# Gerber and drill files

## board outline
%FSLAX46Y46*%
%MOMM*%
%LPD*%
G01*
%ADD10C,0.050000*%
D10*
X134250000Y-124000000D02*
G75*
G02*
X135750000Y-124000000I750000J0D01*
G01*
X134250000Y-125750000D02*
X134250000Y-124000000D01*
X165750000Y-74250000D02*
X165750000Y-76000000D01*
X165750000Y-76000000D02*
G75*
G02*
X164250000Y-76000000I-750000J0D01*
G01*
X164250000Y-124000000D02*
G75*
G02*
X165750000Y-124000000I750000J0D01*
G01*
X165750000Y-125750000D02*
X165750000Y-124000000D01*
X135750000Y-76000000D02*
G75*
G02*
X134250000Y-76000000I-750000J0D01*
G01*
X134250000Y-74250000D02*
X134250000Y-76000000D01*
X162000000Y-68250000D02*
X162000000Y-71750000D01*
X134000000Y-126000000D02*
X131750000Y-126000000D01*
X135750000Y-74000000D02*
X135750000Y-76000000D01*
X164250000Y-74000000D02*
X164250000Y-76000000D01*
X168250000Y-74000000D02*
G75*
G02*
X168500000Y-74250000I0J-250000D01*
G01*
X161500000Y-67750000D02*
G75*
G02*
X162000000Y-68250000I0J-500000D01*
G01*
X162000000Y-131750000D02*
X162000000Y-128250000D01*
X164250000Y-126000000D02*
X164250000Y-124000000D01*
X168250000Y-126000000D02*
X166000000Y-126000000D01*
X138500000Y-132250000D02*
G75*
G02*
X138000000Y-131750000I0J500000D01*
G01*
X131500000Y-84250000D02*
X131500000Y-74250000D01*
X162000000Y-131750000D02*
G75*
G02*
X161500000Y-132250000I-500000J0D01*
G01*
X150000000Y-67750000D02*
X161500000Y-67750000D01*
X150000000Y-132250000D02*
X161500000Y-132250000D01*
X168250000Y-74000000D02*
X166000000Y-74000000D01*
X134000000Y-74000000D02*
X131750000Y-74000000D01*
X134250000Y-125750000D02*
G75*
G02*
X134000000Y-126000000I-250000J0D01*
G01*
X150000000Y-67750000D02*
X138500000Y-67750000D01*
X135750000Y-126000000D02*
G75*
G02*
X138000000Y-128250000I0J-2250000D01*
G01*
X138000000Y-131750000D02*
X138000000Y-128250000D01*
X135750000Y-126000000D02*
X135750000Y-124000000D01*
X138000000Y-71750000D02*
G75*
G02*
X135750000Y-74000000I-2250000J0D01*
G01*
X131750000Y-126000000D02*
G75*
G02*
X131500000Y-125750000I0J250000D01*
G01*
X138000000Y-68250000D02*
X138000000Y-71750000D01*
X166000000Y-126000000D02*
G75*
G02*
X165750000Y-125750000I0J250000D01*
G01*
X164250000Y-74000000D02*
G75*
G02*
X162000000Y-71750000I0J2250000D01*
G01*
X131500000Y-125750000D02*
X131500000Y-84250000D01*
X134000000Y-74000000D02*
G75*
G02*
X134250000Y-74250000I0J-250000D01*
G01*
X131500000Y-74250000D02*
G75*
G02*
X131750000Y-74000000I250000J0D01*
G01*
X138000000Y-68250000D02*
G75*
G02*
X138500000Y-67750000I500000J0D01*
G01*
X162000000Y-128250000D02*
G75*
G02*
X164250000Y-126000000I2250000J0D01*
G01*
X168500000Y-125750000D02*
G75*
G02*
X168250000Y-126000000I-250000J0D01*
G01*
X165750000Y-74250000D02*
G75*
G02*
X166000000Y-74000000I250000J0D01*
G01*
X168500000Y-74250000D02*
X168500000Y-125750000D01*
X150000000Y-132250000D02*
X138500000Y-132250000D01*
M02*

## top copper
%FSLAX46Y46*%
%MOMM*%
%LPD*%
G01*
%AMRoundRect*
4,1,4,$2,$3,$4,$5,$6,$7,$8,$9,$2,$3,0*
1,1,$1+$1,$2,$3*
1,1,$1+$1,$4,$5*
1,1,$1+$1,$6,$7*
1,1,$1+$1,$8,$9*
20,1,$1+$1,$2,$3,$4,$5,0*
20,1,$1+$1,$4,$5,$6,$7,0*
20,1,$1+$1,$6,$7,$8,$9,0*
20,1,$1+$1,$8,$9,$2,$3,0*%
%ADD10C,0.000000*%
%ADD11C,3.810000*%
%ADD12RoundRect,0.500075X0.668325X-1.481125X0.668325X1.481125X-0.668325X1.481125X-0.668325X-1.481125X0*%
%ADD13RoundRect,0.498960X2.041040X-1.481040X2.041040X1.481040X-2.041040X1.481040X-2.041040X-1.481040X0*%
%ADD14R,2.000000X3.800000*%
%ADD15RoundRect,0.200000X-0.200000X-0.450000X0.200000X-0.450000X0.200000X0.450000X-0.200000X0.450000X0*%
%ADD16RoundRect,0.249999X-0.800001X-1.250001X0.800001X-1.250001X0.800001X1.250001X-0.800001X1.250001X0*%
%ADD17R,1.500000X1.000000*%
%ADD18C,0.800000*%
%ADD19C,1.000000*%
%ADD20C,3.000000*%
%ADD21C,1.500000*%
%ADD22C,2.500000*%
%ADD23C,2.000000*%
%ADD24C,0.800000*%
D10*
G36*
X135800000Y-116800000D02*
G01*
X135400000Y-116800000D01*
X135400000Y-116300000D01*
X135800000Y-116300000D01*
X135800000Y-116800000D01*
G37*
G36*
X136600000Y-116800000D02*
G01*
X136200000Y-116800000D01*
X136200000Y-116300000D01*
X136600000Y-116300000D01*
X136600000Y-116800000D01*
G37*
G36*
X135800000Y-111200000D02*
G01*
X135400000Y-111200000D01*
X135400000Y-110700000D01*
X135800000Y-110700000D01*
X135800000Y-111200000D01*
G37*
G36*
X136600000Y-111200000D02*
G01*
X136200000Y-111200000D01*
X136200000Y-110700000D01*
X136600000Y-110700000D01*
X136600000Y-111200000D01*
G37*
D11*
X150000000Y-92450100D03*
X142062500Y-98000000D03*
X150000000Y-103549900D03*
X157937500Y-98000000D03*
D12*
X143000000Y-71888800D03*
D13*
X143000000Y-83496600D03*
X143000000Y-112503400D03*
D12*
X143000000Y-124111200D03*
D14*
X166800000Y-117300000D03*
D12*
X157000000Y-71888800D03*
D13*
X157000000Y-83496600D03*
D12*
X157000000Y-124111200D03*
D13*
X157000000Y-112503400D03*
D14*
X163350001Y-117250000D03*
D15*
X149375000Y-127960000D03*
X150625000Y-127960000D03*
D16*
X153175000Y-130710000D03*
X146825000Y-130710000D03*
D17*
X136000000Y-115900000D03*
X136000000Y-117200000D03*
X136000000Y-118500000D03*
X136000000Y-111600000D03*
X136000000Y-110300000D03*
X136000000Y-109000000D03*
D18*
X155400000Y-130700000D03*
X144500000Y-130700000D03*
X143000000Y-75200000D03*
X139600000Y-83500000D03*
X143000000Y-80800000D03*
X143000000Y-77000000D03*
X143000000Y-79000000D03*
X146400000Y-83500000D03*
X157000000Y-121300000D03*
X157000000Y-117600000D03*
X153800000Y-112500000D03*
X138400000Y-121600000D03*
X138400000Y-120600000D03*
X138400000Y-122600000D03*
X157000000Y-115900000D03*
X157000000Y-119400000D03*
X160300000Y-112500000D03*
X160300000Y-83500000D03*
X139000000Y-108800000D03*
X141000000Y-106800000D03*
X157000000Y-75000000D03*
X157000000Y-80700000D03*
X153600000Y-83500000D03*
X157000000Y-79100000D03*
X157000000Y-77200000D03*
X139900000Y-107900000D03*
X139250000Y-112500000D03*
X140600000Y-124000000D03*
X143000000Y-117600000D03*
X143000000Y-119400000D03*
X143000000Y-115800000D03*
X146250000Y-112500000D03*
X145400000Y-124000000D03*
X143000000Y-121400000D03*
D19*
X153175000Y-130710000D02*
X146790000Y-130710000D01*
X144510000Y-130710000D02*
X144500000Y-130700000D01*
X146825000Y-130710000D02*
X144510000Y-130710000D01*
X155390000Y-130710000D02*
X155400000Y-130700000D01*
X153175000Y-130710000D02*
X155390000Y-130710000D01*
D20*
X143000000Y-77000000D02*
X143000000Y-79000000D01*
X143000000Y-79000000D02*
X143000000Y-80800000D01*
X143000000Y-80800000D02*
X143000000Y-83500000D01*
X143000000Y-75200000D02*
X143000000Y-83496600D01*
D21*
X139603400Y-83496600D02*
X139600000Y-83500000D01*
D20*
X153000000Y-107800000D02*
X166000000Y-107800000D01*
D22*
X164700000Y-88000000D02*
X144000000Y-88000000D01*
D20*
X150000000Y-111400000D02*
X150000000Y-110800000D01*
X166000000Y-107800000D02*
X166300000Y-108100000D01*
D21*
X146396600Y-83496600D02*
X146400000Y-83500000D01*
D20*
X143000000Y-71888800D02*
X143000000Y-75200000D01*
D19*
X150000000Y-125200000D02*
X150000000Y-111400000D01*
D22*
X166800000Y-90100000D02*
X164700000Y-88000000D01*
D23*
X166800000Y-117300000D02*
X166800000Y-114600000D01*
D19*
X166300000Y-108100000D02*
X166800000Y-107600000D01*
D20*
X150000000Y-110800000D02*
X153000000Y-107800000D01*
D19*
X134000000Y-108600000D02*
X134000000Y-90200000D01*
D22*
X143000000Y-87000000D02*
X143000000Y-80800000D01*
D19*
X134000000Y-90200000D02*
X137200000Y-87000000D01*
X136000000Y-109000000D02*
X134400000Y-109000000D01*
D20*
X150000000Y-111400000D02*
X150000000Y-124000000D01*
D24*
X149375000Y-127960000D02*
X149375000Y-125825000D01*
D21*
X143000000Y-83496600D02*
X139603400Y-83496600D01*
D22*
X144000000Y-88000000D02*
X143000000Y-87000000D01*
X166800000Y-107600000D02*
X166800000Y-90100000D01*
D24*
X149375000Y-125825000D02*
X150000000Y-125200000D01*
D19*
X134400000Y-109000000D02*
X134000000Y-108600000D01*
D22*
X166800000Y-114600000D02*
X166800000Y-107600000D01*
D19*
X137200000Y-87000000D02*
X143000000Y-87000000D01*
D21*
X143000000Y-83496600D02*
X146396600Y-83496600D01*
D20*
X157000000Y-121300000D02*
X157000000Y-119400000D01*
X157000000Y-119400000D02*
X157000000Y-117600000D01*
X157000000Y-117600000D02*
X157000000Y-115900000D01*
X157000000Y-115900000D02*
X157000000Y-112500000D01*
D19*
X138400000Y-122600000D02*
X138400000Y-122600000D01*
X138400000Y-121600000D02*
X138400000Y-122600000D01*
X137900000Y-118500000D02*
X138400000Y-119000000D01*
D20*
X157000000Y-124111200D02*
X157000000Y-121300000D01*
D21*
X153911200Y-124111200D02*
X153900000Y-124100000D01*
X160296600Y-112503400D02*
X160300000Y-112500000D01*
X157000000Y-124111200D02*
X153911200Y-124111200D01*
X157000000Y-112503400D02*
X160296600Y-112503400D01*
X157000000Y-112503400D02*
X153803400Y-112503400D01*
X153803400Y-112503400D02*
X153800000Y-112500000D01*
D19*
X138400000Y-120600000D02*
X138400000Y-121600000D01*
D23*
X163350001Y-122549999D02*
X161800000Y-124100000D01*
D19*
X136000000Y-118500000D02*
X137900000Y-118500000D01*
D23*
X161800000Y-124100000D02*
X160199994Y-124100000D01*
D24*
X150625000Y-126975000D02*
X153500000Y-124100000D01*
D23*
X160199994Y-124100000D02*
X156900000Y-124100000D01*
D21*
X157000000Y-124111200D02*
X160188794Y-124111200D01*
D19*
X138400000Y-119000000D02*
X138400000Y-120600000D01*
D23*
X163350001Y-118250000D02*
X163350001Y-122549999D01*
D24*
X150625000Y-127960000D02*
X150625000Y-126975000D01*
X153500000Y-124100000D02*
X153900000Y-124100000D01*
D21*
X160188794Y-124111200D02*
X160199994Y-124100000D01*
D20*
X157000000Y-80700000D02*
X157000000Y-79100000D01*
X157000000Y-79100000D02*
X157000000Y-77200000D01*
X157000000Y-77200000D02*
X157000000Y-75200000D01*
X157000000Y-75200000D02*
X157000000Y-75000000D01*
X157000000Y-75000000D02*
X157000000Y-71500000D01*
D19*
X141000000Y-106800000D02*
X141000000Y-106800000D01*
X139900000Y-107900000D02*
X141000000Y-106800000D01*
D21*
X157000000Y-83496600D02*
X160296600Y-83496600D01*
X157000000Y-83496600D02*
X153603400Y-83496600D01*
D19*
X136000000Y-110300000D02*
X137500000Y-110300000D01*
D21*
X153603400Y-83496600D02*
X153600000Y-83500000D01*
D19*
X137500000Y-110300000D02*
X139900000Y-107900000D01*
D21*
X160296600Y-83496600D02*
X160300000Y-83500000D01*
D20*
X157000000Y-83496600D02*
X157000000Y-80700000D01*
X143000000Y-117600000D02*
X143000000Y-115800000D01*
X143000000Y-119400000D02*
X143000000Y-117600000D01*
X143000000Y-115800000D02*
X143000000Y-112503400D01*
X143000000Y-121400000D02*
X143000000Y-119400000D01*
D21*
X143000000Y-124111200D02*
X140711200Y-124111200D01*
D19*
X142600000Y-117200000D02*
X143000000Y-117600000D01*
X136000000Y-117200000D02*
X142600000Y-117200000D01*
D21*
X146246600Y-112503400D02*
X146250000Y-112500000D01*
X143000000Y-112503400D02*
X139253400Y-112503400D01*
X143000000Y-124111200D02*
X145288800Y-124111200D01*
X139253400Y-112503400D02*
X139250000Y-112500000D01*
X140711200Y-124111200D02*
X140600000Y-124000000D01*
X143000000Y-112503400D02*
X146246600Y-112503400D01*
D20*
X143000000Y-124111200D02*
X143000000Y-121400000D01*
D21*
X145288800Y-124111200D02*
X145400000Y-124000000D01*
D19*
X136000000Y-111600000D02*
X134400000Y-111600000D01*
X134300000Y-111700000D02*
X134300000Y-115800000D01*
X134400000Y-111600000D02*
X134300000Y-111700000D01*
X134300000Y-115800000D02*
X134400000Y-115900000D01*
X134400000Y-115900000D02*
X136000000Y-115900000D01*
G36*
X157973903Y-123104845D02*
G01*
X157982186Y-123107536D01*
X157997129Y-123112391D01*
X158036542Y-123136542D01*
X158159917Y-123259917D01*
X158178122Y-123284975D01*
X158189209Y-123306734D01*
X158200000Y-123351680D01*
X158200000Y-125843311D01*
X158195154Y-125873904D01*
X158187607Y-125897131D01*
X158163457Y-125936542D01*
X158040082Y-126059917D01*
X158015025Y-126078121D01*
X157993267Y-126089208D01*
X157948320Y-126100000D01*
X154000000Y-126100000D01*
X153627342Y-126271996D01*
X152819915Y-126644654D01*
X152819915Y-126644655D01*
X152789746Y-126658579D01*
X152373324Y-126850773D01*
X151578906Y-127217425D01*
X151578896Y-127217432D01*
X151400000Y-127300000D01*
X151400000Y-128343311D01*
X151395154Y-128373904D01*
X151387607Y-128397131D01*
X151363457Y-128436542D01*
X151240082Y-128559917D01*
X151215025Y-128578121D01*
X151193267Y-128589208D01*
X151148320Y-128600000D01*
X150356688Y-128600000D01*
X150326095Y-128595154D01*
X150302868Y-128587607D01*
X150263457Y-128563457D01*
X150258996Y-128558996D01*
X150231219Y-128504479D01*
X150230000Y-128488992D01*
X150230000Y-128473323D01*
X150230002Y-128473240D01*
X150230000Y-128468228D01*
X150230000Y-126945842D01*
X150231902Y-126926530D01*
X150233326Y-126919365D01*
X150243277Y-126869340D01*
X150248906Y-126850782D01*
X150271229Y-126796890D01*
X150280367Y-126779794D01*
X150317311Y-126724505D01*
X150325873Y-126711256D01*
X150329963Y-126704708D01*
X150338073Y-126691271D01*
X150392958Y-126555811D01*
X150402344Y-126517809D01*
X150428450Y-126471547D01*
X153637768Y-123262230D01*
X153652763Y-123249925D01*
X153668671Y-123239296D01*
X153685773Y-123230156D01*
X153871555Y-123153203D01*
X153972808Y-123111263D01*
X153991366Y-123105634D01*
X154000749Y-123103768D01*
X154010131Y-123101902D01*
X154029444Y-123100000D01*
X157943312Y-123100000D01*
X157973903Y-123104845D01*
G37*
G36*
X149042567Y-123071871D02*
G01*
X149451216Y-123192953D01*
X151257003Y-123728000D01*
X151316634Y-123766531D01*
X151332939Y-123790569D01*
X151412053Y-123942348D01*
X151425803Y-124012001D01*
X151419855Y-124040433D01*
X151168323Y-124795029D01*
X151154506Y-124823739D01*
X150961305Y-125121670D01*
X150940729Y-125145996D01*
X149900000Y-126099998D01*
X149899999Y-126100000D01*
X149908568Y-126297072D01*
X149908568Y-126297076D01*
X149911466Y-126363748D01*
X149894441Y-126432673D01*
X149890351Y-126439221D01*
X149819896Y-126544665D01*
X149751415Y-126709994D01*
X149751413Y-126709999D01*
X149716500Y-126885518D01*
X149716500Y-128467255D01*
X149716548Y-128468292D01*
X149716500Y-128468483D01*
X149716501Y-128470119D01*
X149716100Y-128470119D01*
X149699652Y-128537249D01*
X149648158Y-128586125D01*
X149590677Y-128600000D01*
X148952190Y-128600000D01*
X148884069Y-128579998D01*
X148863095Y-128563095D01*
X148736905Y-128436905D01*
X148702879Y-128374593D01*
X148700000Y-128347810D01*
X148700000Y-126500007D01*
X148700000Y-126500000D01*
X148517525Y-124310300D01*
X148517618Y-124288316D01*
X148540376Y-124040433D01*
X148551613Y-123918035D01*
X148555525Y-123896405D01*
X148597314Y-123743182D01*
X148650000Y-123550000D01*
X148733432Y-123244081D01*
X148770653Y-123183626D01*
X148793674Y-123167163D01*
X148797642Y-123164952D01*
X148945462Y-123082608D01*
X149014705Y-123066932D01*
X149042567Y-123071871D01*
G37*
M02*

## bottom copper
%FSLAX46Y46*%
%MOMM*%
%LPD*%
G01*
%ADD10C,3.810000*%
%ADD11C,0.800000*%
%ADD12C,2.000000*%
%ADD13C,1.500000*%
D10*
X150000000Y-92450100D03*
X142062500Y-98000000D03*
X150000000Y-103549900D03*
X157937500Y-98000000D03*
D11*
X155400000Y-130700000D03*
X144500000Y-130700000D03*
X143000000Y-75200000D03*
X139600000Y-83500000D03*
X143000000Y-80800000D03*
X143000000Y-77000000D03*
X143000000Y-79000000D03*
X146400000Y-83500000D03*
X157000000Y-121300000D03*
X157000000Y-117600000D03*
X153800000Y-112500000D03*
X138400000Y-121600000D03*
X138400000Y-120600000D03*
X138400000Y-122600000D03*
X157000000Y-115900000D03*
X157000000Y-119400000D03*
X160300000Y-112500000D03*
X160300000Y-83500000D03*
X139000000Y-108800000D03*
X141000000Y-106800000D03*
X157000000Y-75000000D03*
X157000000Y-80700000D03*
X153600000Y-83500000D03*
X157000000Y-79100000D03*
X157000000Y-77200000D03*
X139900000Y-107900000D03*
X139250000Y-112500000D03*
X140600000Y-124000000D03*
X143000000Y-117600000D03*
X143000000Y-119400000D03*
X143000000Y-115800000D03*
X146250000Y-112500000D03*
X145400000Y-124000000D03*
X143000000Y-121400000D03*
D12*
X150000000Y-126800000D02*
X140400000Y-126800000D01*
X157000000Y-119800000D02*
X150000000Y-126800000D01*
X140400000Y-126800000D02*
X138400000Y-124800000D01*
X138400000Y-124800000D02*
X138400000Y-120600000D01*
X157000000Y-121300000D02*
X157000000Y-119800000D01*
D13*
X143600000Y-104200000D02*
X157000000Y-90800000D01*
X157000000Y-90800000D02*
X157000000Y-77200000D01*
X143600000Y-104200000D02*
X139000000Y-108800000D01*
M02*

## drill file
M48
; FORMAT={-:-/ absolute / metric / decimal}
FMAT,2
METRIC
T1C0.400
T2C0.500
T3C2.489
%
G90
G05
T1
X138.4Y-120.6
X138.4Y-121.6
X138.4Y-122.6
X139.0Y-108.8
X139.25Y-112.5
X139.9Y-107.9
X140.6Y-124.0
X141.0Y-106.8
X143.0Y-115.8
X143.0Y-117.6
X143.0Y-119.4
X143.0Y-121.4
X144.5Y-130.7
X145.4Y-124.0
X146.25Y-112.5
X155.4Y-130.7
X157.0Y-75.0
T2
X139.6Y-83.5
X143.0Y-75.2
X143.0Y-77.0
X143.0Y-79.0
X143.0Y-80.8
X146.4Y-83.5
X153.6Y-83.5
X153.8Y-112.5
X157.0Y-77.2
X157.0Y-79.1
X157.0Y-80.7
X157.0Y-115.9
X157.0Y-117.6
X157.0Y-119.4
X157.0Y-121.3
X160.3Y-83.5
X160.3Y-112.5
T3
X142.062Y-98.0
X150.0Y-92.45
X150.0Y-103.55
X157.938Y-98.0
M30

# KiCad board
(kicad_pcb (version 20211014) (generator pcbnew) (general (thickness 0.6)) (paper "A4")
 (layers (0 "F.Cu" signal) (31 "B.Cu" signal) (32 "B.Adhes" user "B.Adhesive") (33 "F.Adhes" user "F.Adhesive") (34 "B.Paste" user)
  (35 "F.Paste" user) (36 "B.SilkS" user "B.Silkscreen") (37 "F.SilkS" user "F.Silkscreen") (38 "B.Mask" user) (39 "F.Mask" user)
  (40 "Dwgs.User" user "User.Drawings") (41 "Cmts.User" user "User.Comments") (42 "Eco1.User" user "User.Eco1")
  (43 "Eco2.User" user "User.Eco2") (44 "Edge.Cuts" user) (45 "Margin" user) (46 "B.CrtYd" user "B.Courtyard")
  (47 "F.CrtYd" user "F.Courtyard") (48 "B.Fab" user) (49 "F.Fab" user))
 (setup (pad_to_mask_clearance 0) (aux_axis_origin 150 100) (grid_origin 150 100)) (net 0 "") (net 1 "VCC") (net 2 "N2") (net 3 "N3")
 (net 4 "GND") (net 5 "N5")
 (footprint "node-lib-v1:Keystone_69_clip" (layer "F.Cu") (at 150 98 180)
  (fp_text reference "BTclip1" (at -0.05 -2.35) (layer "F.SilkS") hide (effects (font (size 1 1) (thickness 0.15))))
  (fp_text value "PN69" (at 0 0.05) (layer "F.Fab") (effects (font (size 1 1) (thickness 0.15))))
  (pad "" smd circle locked (at 0 -5.5499 180) (size 3.81 3.81) (layers "F.Paste" "F.Mask"))
  (pad "" smd circle locked (at -7.9375 0 180) (size 3.81 3.81) (layers "F.Paste" "F.Mask"))
  (pad "" smd circle locked (at 7.9375 0 180) (size 3.81 3.81) (layers "F.Paste" "F.Mask"))
  (pad "" smd circle locked (at 0 5.5499 180) (size 3.81 3.81) (layers "F.Paste" "F.Mask"))
  (pad "1" thru_hole circle locked (at 0 5.5499 180) (size 3.81 3.81) (drill 2.4892) (layers *.Cu *.Mask))
  (pad "1" thru_hole circle locked (at 7.9375 0 180) (size 3.81 3.81) (drill 2.4892) (layers *.Cu *.Mask))
  (pad "1" thru_hole circle locked (at 0 -5.5499 180) (size 3.81 3.81) (drill 2.4892) (layers *.Cu *.Mask))
  (pad "1" thru_hole circle locked (at -7.9375 0 180) (size 3.81 3.81) (drill 2.4892) (layers *.Cu *.Mask "F.Paste")))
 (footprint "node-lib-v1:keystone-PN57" (layer "F.Cu") (at 143 98 90)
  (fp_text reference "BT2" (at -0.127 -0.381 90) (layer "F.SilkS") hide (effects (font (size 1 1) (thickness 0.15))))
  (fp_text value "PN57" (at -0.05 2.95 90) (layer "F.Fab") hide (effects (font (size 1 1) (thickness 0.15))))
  (pad "1" smd roundrect locked (at 26.1112 0 90) (size 3.9624 2.3368) (layers "F.Cu" "F.Paste" "F.Mask") (roundrect_rratio 0.2139999144)
   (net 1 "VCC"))
  (pad "1" smd roundrect locked (at 14.5034 0 90) (size 3.96 5.08) (layers "F.Cu" "F.Paste" "F.Mask") (roundrect_rratio 0.126) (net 1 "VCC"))
  (pad "2" smd roundrect locked (at -14.5034 0 90) (size 3.96 5.08) (layers "F.Cu" "F.Paste" "F.Mask") (roundrect_rratio 0.126) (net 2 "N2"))
  (pad "2" smd roundrect locked (at -26.1112 0 90) (size 3.9624 2.3368) (layers "F.Cu" "F.Paste" "F.Mask") (roundrect_rratio 0.2139999144)
   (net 2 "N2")))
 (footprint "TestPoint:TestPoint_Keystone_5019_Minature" (layer "F.Cu") (at 166.8 117.3 -90)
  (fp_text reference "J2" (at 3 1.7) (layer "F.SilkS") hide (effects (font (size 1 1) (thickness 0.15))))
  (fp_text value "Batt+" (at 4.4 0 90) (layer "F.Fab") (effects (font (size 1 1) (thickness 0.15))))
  (pad "1" smd rect locked (at 0 0 270) (size 3.8 2) (layers "F.Cu" "F.Mask") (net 1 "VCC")))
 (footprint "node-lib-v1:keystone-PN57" (layer "F.Cu") (at 157 98 90)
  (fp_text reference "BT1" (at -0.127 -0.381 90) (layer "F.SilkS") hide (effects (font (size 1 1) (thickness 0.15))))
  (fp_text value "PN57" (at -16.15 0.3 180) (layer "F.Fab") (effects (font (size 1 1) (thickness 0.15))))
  (pad "1" smd roundrect locked (at 26.1112 0 90) (size 3.9624 2.3368) (layers "F.Cu" "F.Paste" "F.Mask") (roundrect_rratio 0.2139999144)
   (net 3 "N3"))
  (pad "1" smd roundrect locked (at 14.5034 0 90) (size 3.96 5.08) (layers "F.Cu" "F.Paste" "F.Mask") (roundrect_rratio 0.126) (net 3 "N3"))
  (pad "2" smd roundrect locked (at -26.1112 0 90) (size 3.9624 2.3368) (layers "F.Cu" "F.Paste" "F.Mask") (roundrect_rratio 0.2139999144)
   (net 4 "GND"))
  (pad "2" smd roundrect locked (at -14.5034 0 90) (size 3.96 5.08) (layers "F.Cu" "F.Paste" "F.Mask") (roundrect_rratio 0.126)
   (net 4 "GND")))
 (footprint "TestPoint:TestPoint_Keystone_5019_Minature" (layer "F.Cu") (at 163.350001 117.25 90)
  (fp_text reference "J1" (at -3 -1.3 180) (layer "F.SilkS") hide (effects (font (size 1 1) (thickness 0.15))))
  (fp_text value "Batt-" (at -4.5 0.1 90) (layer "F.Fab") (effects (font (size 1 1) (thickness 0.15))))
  (pad "1" smd rect locked (at 0 0 90) (size 3.8 2) (layers "F.Cu" "F.Mask") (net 4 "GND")))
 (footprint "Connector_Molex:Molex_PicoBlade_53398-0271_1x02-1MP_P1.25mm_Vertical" (layer "F.Cu") (at 150 129.21)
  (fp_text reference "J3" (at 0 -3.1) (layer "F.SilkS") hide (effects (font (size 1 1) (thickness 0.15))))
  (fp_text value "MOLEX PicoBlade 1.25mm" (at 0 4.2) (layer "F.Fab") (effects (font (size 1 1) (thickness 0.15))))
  (pad "1" smd roundrect locked (at -0.625 -1.25) (size 0.8 1.3) (layers "F.Cu" "F.Paste" "F.Mask") (roundrect_rratio 0.25) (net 1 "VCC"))
  (pad "2" smd roundrect locked (at 0.625 -1.25) (size 0.8 1.3) (layers "F.Cu" "F.Paste" "F.Mask") (roundrect_rratio 0.25) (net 4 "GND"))
  (pad "MP" smd roundrect locked (at 3.175 1.5) (size 2.1 3) (layers "F.Cu" "F.Paste" "F.Mask") (roundrect_rratio 0.1190471429))
  (pad "MP" smd roundrect locked (at -3.175 1.5) (size 2.1 3) (layers "F.Cu" "F.Paste" "F.Mask") (roundrect_rratio 0.1190471429)))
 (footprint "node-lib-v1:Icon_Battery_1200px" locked (layer "F.Cu") (at 135 82.75)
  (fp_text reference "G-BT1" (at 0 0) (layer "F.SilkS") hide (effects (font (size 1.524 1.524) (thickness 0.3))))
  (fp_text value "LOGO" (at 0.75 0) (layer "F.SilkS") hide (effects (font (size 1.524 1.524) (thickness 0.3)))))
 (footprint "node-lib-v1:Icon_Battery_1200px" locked (layer "F.Cu") (at 165 82.5)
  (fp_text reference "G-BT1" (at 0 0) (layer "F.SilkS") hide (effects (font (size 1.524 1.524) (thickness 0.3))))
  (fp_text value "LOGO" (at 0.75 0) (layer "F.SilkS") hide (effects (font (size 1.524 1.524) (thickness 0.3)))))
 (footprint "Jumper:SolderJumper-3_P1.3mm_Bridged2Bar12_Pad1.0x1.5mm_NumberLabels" (layer "F.Cu") (at 136 117.2 -90)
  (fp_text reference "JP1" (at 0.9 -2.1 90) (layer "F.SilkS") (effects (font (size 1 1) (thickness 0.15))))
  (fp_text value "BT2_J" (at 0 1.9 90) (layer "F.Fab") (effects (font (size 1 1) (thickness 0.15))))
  (fp_poly (pts (xy -0.9 0.2) (xy -0.4 0.2) (xy -0.4 0.6) (xy -0.9 0.6)) (layer "F.Cu") (width 0) (fill solid))
  (fp_poly (pts (xy -0.9 -0.6) (xy -0.4 -0.6) (xy -0.4 -0.2) (xy -0.9 -0.2)) (layer "F.Cu") (width 0) (fill solid))
  (pad "1" smd rect locked (at -1.3 0 270) (size 1 1.5) (layers "F.Cu" "F.Mask") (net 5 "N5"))
  (pad "2" smd rect locked (at 0 0 270) (size 1 1.5) (layers "F.Cu" "F.Mask") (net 2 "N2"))
  (pad "3" smd rect locked (at 1.3 0 270) (size 1 1.5) (layers "F.Cu" "F.Mask") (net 4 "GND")))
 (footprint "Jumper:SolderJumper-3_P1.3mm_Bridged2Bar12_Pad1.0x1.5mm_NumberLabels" (layer "F.Cu") (at 136 110.3 90)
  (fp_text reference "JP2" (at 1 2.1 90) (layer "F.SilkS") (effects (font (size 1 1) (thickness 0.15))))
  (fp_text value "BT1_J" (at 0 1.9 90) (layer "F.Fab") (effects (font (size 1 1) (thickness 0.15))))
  (fp_poly (pts (xy -0.9 -0.6) (xy -0.4 -0.6) (xy -0.4 -0.2) (xy -0.9 -0.2)) (layer "F.Cu") (width 0) (fill solid))
  (fp_poly (pts (xy -0.9 0.2) (xy -0.4 0.2) (xy -0.4 0.6) (xy -0.9 0.6)) (layer "F.Cu") (width 0) (fill solid))
  (pad "1" smd rect locked (at -1.3 0 90) (size 1 1.5) (layers "F.Cu" "F.Mask") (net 5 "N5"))
  (pad "2" smd rect locked (at 0 0 90) (size 1 1.5) (layers "F.Cu" "F.Mask") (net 3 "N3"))
  (pad "3" smd rect locked (at 1.3 0 90) (size 1 1.5) (layers "F.Cu" "F.Mask") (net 1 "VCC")))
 (gr_arc (start 134.25 124) (mid 135 123.25) (end 135.75 124) (layer "Edge.Cuts") (width 0.05))
 (gr_line (start 134.25 125.75) (end 134.25 124) (layer "Edge.Cuts") (width 0.05))
 (gr_line (start 165.75 74.25) (end 165.75 76) (layer "Edge.Cuts") (width 0.05))
 (gr_arc (start 165.75 76) (mid 165 76.75) (end 164.25 76) (layer "Edge.Cuts") (width 0.05))
 (gr_arc (start 164.25 124) (mid 165 123.25) (end 165.75 124) (layer "Edge.Cuts") (width 0.05))
 (gr_line (start 165.75 125.75) (end 165.75 124) (layer "Edge.Cuts") (width 0.05))
 (gr_arc (start 135.75 76) (mid 135 76.75) (end 134.25 76) (layer "Edge.Cuts") (width 0.05))
 (gr_line (start 134.25 74.25) (end 134.25 76) (layer "Edge.Cuts") (width 0.05))
 (gr_line (start 162 68.25) (end 162 71.75) (layer "Edge.Cuts") (width 0.05))
 (gr_line (start 134 126) (end 131.75 126) (layer "Edge.Cuts") (width 0.05))
 (gr_line (start 135.75 74) (end 135.75 76) (layer "Edge.Cuts") (width 0.05))
 (gr_line (start 164.25 74) (end 164.25 76) (layer "Edge.Cuts") (width 0.05))
 (gr_arc (start 168.25 74) (mid 168.426777 74.073223) (end 168.5 74.25) (layer "Edge.Cuts") (width 0.05))
 (gr_arc (start 161.5 67.75) (mid 161.853553 67.896447) (end 162 68.25) (layer "Edge.Cuts") (width 0.05))
 (gr_line (start 162 131.75) (end 162 128.25) (layer "Edge.Cuts") (width 0.05))
 (gr_line (start 164.25 126) (end 164.25 124) (layer "Edge.Cuts") (width 0.05))
 (gr_line (start 168.25 126) (end 166 126) (layer "Edge.Cuts") (width 0.05))
 (gr_arc (start 138.5 132.25) (mid 138.146447 132.103553) (end 138 131.75) (layer "Edge.Cuts") (width 0.05))
 (gr_line (start 131.5 84.25) (end 131.5 74.25) (layer "Edge.Cuts") (width 0.05))
 (gr_arc (start 162 131.75) (mid 161.853553 132.103553) (end 161.5 132.25) (layer "Edge.Cuts") (width 0.05))
 (gr_line (start 150 67.75) (end 161.5 67.75) (layer "Edge.Cuts") (width 0.05))
 (gr_line (start 150 132.25) (end 161.5 132.25) (layer "Edge.Cuts") (width 0.05))
 (gr_line (start 168.25 74) (end 166 74) (layer "Edge.Cuts") (width 0.05))
 (gr_line (start 134 74) (end 131.75 74) (layer "Edge.Cuts") (width 0.05))
 (gr_arc (start 134.25 125.75) (mid 134.176777 125.926777) (end 134 126) (layer "Edge.Cuts") (width 0.05))
 (gr_line (start 150 67.75) (end 138.5 67.75) (layer "Edge.Cuts") (width 0.05))
 (gr_arc (start 135.75 126) (mid 137.34099 126.65901) (end 138 128.25) (layer "Edge.Cuts") (width 0.05))
 (gr_line (start 138 131.75) (end 138 128.25) (layer "Edge.Cuts") (width 0.05))
 (gr_line (start 135.75 126) (end 135.75 124) (layer "Edge.Cuts") (width 0.05))
 (gr_arc (start 138 71.75) (mid 137.34099 73.34099) (end 135.75 74) (layer "Edge.Cuts") (width 0.05))
 (gr_arc (start 131.75 126) (mid 131.573223 125.926777) (end 131.5 125.75) (layer "Edge.Cuts") (width 0.05))
 (gr_line (start 138 68.25) (end 138 71.75) (layer "Edge.Cuts") (width 0.05))
 (gr_arc (start 166 126) (mid 165.823223 125.926777) (end 165.75 125.75) (layer "Edge.Cuts") (width 0.05))
 (gr_arc (start 164.25 74) (mid 162.65901 73.34099) (end 162 71.75) (layer "Edge.Cuts") (width 0.05))
 (gr_line (start 131.5 125.75) (end 131.5 84.25) (layer "Edge.Cuts") (width 0.05))
 (gr_arc (start 134 74) (mid 134.176777 74.073223) (end 134.25 74.25) (layer "Edge.Cuts") (width 0.05))
 (gr_arc (start 131.5 74.25) (mid 131.573223 74.073223) (end 131.75 74) (layer "Edge.Cuts") (width 0.05))
 (gr_arc (start 138 68.25) (mid 138.146447 67.896447) (end 138.5 67.75) (layer "Edge.Cuts") (width 0.05))
 (gr_arc (start 162 128.25) (mid 162.65901 126.65901) (end 164.25 126) (layer "Edge.Cuts") (width 0.05))
 (gr_arc (start 168.5 125.75) (mid 168.426777 125.926777) (end 168.25 126) (layer "Edge.Cuts") (width 0.05))
 (gr_arc (start 165.75 74.25) (mid 165.823223 74.073223) (end 166 74) (layer "Edge.Cuts") (width 0.05))
 (gr_line (start 168.5 74.25) (end 168.5 125.75) (layer "Edge.Cuts") (width 0.05))
 (gr_line (start 150 132.25) (end 138.5 132.25) (layer "Edge.Cuts") (width 0.05))
 (segment (start 153.175 130.71) (end 146.79 130.71) (width 1) (layer "F.Cu") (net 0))
 (segment (start 144.51 130.71) (end 144.5 130.7) (width 1) (layer "F.Cu") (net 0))
 (segment (start 146.825 130.71) (end 144.51 130.71) (width 1) (layer "F.Cu") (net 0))
 (segment (start 155.39 130.71) (end 155.4 130.7) (width 1) (layer "F.Cu") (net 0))
 (segment (start 153.175 130.71) (end 155.39 130.71) (width 1) (layer "F.Cu") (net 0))
 (via (at 155.4 130.7) (size 0.8) (drill 0.4) (layers "F.Cu" "B.Cu") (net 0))
 (via (at 144.5 130.7) (size 0.8) (drill 0.4) (layers "F.Cu" "B.Cu") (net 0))
 (segment (start 143 77) (end 143 79) (width 3) (layer "F.Cu") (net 1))
 (segment (start 143 79) (end 143 80.8) (width 3) (layer "F.Cu") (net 1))
 (segment (start 143 80.8) (end 143 83.5) (width 3) (layer "F.Cu") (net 1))
 (segment (start 143 75.2) (end 143 83.4966) (width 3) (layer "F.Cu") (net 1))
 (segment (start 139.6034 83.4966) (end 139.6 83.5) (width 1.5) (layer "F.Cu") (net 1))
 (segment (start 153 107.8) (end 166 107.8) (width 3) (layer "F.Cu") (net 1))
 (segment (start 164.7 88) (end 144 88) (width 2.5) (layer "F.Cu") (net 1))
 (segment (start 150 111.4) (end 150 110.8) (width 3) (layer "F.Cu") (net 1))
 (segment (start 166 107.8) (end 166.3 108.1) (width 3) (layer "F.Cu") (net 1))
 (segment (start 146.3966 83.4966) (end 146.4 83.5) (width 1.5) (layer "F.Cu") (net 1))
 (segment (start 143 71.8888) (end 143 75.2) (width 3) (layer "F.Cu") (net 1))
 (segment (start 150 125.2) (end 150 111.4) (width 1) (layer "F.Cu") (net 1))
 (segment (start 166.8 90.1) (end 164.7 88) (width 2.5) (layer "F.Cu") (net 1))
 (segment (start 166.8 117.3) (end 166.8 114.6) (width 2) (layer "F.Cu") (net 1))
 (segment (start 166.3 108.1) (end 166.8 107.6) (width 1) (layer "F.Cu") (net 1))
 (segment (start 150 110.8) (end 153 107.8) (width 3) (layer "F.Cu") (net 1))
 (segment (start 134 108.6) (end 134 90.2) (width 1) (layer "F.Cu") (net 1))
 (segment (start 143 87) (end 143 80.8) (width 2.5) (layer "F.Cu") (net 1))
 (segment (start 134 90.2) (end 137.2 87) (width 1) (layer "F.Cu") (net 1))
 (segment (start 136 109) (end 134.4 109) (width 1) (layer "F.Cu") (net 1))
 (segment (start 150 111.4) (end 150 124) (width 3) (layer "F.Cu") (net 1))
 (segment (start 149.375 127.96) (end 149.375 125.825) (width 0.8) (layer "F.Cu") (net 1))
 (segment (start 143 83.4966) (end 139.6034 83.4966) (width 1.5) (layer "F.Cu") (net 1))
 (segment (start 144 88) (end 143 87) (width 2.5) (layer "F.Cu") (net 1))
 (segment (start 166.8 107.6) (end 166.8 90.1) (width 2.5) (layer "F.Cu") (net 1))
 (segment (start 149.375 125.825) (end 150 125.2) (width 0.8) (layer "F.Cu") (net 1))
 (segment (start 134.4 109) (end 134 108.6) (width 1) (layer "F.Cu") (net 1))
 (segment (start 166.8 114.6) (end 166.8 107.6) (width 2.5) (layer "F.Cu") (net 1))
 (segment (start 137.2 87) (end 143 87) (width 1) (layer "F.Cu") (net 1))
 (segment (start 143 83.4966) (end 146.3966 83.4966) (width 1.5) (layer "F.Cu") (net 1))
 (via (at 143 75.2) (size 0.8) (drill 0.5) (layers "F.Cu" "B.Cu") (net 1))
 (via (at 139.6 83.5) (size 0.8) (drill 0.5) (layers "F.Cu" "B.Cu") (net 1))
 (via (at 143 80.8) (size 0.8) (drill 0.5) (layers "F.Cu" "B.Cu") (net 1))
 (via (at 143 77) (size 0.8) (drill 0.5) (layers "F.Cu" "B.Cu") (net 1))
 (via (at 143 79) (size 0.8) (drill 0.5) (layers "F.Cu" "B.Cu") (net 1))
 (via (at 146.4 83.5) (size 0.8) (drill 0.5) (layers "F.Cu" "B.Cu") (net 1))
 (segment (start 157 121.3) (end 157 119.4) (width 3) (layer "F.Cu") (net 4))
 (segment (start 157 119.4) (end 157 117.6) (width 3) (layer "F.Cu") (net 4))
 (segment (start 157 117.6) (end 157 115.9) (width 3) (layer "F.Cu") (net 4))
 (segment (start 157 115.9) (end 157 112.5) (width 3) (layer "F.Cu") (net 4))
 (segment (start 138.4 122.6) (end 138.4 122.6) (width 1) (layer "F.Cu") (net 4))
 (segment (start 138.4 121.6) (end 138.4 122.6) (width 1) (layer "F.Cu") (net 4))
 (segment (start 137.9 118.5) (end 138.4 119) (width 1) (layer "F.Cu") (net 4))
 (segment (start 157 124.1112) (end 157 121.3) (width 3) (layer "F.Cu") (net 4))
 (segment (start 153.9112 124.1112) (end 153.9 124.1) (width 1.5) (layer "F.Cu") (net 4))
 (segment (start 160.2966 112.5034) (end 160.3 112.5) (width 1.5) (layer "F.Cu") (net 4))
 (segment (start 157 124.1112) (end 153.9112 124.1112) (width 1.5) (layer "F.Cu") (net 4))
 (segment (start 157 112.5034) (end 160.2966 112.5034) (width 1.5) (layer "F.Cu") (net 4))
 (segment (start 157 112.5034) (end 153.8034 112.5034) (width 1.5) (layer "F.Cu") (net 4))
 (segment (start 153.8034 112.5034) (end 153.8 112.5) (width 1.5) (layer "F.Cu") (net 4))
 (segment (start 138.4 120.6) (end 138.4 121.6) (width 1) (layer "F.Cu") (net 4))
 (segment (start 163.350001 122.549999) (end 161.8 124.1) (width 2) (layer "F.Cu") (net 4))
 (segment (start 136 118.5) (end 137.9 118.5) (width 1) (layer "F.Cu") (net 4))
 (segment (start 161.8 124.1) (end 160.199994 124.1) (width 2) (layer "F.Cu") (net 4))
 (segment (start 150.625 126.975) (end 153.5 124.1) (width 0.8) (layer "F.Cu") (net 4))
 (segment (start 160.199994 124.1) (end 156.9 124.1) (width 2) (layer "F.Cu") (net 4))
 (segment (start 157 124.1112) (end 160.188794 124.1112) (width 1.5) (layer "F.Cu") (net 4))
 (segment (start 138.4 119) (end 138.4 120.6) (width 1) (layer "F.Cu") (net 4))
 (segment (start 163.350001 118.25) (end 163.350001 122.549999) (width 2) (layer "F.Cu") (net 4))
 (segment (start 150.625 127.96) (end 150.625 126.975) (width 0.8) (layer "F.Cu") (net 4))
 (segment (start 153.5 124.1) (end 153.9 124.1) (width 0.8) (layer "F.Cu") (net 4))
 (segment (start 160.188794 124.1112) (end 160.199994 124.1) (width 1.5) (layer "F.Cu") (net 4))
 (via (at 157 121.3) (size 0.8) (drill 0.5) (layers "F.Cu" "B.Cu") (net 4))
 (via (at 157 117.6) (size 0.8) (drill 0.5) (layers "F.Cu" "B.Cu") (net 4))
 (via (at 153.8 112.5) (size 0.8) (drill 0.5) (layers "F.Cu" "B.Cu") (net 4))
 (via (at 138.4 121.6) (size 0.8) (drill 0.4) (layers "F.Cu" "B.Cu") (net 4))
 (via (at 138.4 120.6) (size 0.8) (drill 0.4) (layers "F.Cu" "B.Cu") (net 4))
 (via (at 138.4 122.6) (size 0.8) (drill 0.4) (layers "F.Cu" "B.Cu") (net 4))
 (via (at 157 115.9) (size 0.8) (drill 0.5) (layers "F.Cu" "B.Cu") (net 4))
 (via (at 157 119.4) (size 0.8) (drill 0.5) (layers "F.Cu" "B.Cu") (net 4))
 (via (at 160.3 112.5) (size 0.8) (drill 0.5) (layers "F.Cu" "B.Cu") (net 4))
 (segment (start 150 126.8) (end 140.4 126.8) (width 2) (layer "B.Cu") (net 4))
 (segment (start 157 119.8) (end 150 126.8) (width 2) (layer "B.Cu") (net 4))
 (segment (start 140.4 126.8) (end 138.4 124.8) (width 2) (layer "B.Cu") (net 4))
 (segment (start 138.4 124.8) (end 138.4 120.6) (width 2) (layer "B.Cu") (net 4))
 (segment (start 157 121.3) (end 157 119.8) (width 2) (layer "B.Cu") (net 4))
 (segment (start 157 80.7) (end 157 79.1) (width 3) (layer "F.Cu") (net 3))
 (segment (start 157 79.1) (end 157 77.2) (width 3) (layer "F.Cu") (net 3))
 (segment (start 157 77.2) (end 157 75.2) (width 3) (layer "F.Cu") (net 3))
 (segment (start 157 75.2) (end 157 75) (width 3) (layer "F.Cu") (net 3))
 (segment (start 157 75) (end 157 71.5) (width 3) (layer "F.Cu") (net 3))
 (segment (start 141 106.8) (end 141 106.8) (width 1) (layer "F.Cu") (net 3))
 (segment (start 139.9 107.9) (end 141 106.8) (width 1) (layer "F.Cu") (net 3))
 (segment (start 157 83.4966) (end 160.2966 83.4966) (width 1.5) (layer "F.Cu") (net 3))
 (segment (start 157 83.4966) (end 153.6034 83.4966) (width 1.5) (layer "F.Cu") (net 3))
 (segment (start 136 110.3) (end 137.5 110.3) (width 1) (layer "F.Cu") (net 3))
 (segment (start 153.6034 83.4966) (end 153.6 83.5) (width 1.5) (layer "F.Cu") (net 3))
 (segment (start 137.5 110.3) (end 139.9 107.9) (width 1) (layer "F.Cu") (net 3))
 (segment (start 160.2966 83.4966) (end 160.3 83.5) (width 1.5) (layer "F.Cu") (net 3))
 (segment (start 157 83.4966) (end 157 80.7) (width 3) (layer "F.Cu") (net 3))
 (via (at 160.3 83.5) (size 0.8) (drill 0.5) (layers "F.Cu" "B.Cu") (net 3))
 (via (at 139 108.8) (size 0.8) (drill 0.4) (layers "F.Cu" "B.Cu") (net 3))
 (via (at 141 106.8) (size 0.8) (drill 0.4) (layers "F.Cu" "B.Cu") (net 3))
 (via (at 157 75) (size 0.8) (drill 0.4) (layers "F.Cu" "B.Cu") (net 3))
 (via (at 157 80.7) (size 0.8) (drill 0.5) (layers "F.Cu" "B.Cu") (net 3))
 (via (at 153.6 83.5) (size 0.8) (drill 0.5) (layers "F.Cu" "B.Cu") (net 3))
 (via (at 157 79.1) (size 0.8) (drill 0.5) (layers "F.Cu" "B.Cu") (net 3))
 (via (at 157 77.2) (size 0.8) (drill 0.5) (layers "F.Cu" "B.Cu") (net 3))
 (via (at 139.9 107.9) (size 0.8) (drill 0.4) (layers "F.Cu" "B.Cu") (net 3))
 (segment (start 143.6 104.2) (end 157 90.8) (width 1.5) (layer "B.Cu") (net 3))
 (segment (start 157 90.8) (end 157 77.2) (width 1.5) (layer "B.Cu") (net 3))
 (segment (start 143.6 104.2) (end 139 108.8) (width 1.5) (layer "B.Cu") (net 3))
 (segment (start 143 117.6) (end 143 115.8) (width 3) (layer "F.Cu") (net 2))
 (segment (start 143 119.4) (end 143 117.6) (width 3) (layer "F.Cu") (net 2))
 (segment (start 143 115.8) (end 143 112.5034) (width 3) (layer "F.Cu") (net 2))
 (segment (start 143 121.4) (end 143 119.4) (width 3) (layer "F.Cu") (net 2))
 (segment (start 143 124.1112) (end 140.7112 124.1112) (width 1.5) (layer "F.Cu") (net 2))
 (segment (start 142.6 117.2) (end 143 117.6) (width 1) (layer "F.Cu") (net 2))
 (segment (start 136 117.2) (end 142.6 117.2) (width 1) (layer "F.Cu") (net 2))
 (segment (start 146.2466 112.5034) (end 146.25 112.5) (width 1.5) (layer "F.Cu") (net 2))
 (segment (start 143 112.5034) (end 139.2534 112.5034) (width 1.5) (layer "F.Cu") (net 2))
 (segment (start 143 124.1112) (end 145.2888 124.1112) (width 1.5) (layer "F.Cu") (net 2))
 (segment (start 139.2534 112.5034) (end 139.25 112.5) (width 1.5) (layer "F.Cu") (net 2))
 (segment (start 140.7112 124.1112) (end 140.6 124) (width 1.5) (layer "F.Cu") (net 2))
 (segment (start 143 112.5034) (end 146.2466 112.5034) (width 1.5) (layer "F.Cu") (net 2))
 (segment (start 143 124.1112) (end 143 121.4) (width 3) (layer "F.Cu") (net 2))
 (segment (start 145.2888 124.1112) (end 145.4 124) (width 1.5) (layer "F.Cu") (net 2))
 (via (at 139.25 112.5) (size 0.8) (drill 0.4) (layers "F.Cu" "B.Cu") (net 2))
 (via (at 140.6 124) (size 0.8) (drill 0.4) (layers "F.Cu" "B.Cu") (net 2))
 (via (at 143 117.6) (size 0.8) (drill 0.4) (layers "F.Cu" "B.Cu") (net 2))
 (via (at 143 119.4) (size 0.8) (drill 0.4) (layers "F.Cu" "B.Cu") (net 2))
 (via (at 143 115.8) (size 0.8) (drill 0.4) (layers "F.Cu" "B.Cu") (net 2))
 (via (at 146.25 112.5) (size 0.8) (drill 0.4) (layers "F.Cu" "B.Cu") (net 2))
 (via (at 145.4 124) (size 0.8) (drill 0.4) (layers "F.Cu" "B.Cu") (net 2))
 (via (at 143 121.4) (size 0.8) (drill 0.4) (layers "F.Cu" "B.Cu") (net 2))
 (segment (start 136 111.6) (end 134.4 111.6) (width 1) (layer "F.Cu") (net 5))
 (segment (start 134.3 111.7) (end 134.3 115.8) (width 1) (layer "F.Cu") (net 5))
 (segment (start 134.4 111.6) (end 134.3 111.7) (width 1) (layer "F.Cu") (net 5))
 (segment (start 134.3 115.8) (end 134.4 115.9) (width 1) (layer "F.Cu") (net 5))
 (segment (start 134.4 115.9) (end 136 115.9) (width 1) (layer "F.Cu") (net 5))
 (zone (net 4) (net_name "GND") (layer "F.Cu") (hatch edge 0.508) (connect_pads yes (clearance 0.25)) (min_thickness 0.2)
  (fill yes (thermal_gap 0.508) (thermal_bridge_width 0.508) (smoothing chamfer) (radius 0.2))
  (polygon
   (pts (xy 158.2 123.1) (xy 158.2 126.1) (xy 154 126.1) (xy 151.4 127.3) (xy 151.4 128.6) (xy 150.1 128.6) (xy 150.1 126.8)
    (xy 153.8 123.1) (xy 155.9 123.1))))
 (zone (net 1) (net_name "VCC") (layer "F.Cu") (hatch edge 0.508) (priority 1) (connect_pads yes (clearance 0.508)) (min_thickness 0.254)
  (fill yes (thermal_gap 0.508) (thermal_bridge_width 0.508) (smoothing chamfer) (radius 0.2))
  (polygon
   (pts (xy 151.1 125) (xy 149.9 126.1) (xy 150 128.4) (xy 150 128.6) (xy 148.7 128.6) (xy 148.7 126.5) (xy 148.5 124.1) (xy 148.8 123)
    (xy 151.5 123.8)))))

